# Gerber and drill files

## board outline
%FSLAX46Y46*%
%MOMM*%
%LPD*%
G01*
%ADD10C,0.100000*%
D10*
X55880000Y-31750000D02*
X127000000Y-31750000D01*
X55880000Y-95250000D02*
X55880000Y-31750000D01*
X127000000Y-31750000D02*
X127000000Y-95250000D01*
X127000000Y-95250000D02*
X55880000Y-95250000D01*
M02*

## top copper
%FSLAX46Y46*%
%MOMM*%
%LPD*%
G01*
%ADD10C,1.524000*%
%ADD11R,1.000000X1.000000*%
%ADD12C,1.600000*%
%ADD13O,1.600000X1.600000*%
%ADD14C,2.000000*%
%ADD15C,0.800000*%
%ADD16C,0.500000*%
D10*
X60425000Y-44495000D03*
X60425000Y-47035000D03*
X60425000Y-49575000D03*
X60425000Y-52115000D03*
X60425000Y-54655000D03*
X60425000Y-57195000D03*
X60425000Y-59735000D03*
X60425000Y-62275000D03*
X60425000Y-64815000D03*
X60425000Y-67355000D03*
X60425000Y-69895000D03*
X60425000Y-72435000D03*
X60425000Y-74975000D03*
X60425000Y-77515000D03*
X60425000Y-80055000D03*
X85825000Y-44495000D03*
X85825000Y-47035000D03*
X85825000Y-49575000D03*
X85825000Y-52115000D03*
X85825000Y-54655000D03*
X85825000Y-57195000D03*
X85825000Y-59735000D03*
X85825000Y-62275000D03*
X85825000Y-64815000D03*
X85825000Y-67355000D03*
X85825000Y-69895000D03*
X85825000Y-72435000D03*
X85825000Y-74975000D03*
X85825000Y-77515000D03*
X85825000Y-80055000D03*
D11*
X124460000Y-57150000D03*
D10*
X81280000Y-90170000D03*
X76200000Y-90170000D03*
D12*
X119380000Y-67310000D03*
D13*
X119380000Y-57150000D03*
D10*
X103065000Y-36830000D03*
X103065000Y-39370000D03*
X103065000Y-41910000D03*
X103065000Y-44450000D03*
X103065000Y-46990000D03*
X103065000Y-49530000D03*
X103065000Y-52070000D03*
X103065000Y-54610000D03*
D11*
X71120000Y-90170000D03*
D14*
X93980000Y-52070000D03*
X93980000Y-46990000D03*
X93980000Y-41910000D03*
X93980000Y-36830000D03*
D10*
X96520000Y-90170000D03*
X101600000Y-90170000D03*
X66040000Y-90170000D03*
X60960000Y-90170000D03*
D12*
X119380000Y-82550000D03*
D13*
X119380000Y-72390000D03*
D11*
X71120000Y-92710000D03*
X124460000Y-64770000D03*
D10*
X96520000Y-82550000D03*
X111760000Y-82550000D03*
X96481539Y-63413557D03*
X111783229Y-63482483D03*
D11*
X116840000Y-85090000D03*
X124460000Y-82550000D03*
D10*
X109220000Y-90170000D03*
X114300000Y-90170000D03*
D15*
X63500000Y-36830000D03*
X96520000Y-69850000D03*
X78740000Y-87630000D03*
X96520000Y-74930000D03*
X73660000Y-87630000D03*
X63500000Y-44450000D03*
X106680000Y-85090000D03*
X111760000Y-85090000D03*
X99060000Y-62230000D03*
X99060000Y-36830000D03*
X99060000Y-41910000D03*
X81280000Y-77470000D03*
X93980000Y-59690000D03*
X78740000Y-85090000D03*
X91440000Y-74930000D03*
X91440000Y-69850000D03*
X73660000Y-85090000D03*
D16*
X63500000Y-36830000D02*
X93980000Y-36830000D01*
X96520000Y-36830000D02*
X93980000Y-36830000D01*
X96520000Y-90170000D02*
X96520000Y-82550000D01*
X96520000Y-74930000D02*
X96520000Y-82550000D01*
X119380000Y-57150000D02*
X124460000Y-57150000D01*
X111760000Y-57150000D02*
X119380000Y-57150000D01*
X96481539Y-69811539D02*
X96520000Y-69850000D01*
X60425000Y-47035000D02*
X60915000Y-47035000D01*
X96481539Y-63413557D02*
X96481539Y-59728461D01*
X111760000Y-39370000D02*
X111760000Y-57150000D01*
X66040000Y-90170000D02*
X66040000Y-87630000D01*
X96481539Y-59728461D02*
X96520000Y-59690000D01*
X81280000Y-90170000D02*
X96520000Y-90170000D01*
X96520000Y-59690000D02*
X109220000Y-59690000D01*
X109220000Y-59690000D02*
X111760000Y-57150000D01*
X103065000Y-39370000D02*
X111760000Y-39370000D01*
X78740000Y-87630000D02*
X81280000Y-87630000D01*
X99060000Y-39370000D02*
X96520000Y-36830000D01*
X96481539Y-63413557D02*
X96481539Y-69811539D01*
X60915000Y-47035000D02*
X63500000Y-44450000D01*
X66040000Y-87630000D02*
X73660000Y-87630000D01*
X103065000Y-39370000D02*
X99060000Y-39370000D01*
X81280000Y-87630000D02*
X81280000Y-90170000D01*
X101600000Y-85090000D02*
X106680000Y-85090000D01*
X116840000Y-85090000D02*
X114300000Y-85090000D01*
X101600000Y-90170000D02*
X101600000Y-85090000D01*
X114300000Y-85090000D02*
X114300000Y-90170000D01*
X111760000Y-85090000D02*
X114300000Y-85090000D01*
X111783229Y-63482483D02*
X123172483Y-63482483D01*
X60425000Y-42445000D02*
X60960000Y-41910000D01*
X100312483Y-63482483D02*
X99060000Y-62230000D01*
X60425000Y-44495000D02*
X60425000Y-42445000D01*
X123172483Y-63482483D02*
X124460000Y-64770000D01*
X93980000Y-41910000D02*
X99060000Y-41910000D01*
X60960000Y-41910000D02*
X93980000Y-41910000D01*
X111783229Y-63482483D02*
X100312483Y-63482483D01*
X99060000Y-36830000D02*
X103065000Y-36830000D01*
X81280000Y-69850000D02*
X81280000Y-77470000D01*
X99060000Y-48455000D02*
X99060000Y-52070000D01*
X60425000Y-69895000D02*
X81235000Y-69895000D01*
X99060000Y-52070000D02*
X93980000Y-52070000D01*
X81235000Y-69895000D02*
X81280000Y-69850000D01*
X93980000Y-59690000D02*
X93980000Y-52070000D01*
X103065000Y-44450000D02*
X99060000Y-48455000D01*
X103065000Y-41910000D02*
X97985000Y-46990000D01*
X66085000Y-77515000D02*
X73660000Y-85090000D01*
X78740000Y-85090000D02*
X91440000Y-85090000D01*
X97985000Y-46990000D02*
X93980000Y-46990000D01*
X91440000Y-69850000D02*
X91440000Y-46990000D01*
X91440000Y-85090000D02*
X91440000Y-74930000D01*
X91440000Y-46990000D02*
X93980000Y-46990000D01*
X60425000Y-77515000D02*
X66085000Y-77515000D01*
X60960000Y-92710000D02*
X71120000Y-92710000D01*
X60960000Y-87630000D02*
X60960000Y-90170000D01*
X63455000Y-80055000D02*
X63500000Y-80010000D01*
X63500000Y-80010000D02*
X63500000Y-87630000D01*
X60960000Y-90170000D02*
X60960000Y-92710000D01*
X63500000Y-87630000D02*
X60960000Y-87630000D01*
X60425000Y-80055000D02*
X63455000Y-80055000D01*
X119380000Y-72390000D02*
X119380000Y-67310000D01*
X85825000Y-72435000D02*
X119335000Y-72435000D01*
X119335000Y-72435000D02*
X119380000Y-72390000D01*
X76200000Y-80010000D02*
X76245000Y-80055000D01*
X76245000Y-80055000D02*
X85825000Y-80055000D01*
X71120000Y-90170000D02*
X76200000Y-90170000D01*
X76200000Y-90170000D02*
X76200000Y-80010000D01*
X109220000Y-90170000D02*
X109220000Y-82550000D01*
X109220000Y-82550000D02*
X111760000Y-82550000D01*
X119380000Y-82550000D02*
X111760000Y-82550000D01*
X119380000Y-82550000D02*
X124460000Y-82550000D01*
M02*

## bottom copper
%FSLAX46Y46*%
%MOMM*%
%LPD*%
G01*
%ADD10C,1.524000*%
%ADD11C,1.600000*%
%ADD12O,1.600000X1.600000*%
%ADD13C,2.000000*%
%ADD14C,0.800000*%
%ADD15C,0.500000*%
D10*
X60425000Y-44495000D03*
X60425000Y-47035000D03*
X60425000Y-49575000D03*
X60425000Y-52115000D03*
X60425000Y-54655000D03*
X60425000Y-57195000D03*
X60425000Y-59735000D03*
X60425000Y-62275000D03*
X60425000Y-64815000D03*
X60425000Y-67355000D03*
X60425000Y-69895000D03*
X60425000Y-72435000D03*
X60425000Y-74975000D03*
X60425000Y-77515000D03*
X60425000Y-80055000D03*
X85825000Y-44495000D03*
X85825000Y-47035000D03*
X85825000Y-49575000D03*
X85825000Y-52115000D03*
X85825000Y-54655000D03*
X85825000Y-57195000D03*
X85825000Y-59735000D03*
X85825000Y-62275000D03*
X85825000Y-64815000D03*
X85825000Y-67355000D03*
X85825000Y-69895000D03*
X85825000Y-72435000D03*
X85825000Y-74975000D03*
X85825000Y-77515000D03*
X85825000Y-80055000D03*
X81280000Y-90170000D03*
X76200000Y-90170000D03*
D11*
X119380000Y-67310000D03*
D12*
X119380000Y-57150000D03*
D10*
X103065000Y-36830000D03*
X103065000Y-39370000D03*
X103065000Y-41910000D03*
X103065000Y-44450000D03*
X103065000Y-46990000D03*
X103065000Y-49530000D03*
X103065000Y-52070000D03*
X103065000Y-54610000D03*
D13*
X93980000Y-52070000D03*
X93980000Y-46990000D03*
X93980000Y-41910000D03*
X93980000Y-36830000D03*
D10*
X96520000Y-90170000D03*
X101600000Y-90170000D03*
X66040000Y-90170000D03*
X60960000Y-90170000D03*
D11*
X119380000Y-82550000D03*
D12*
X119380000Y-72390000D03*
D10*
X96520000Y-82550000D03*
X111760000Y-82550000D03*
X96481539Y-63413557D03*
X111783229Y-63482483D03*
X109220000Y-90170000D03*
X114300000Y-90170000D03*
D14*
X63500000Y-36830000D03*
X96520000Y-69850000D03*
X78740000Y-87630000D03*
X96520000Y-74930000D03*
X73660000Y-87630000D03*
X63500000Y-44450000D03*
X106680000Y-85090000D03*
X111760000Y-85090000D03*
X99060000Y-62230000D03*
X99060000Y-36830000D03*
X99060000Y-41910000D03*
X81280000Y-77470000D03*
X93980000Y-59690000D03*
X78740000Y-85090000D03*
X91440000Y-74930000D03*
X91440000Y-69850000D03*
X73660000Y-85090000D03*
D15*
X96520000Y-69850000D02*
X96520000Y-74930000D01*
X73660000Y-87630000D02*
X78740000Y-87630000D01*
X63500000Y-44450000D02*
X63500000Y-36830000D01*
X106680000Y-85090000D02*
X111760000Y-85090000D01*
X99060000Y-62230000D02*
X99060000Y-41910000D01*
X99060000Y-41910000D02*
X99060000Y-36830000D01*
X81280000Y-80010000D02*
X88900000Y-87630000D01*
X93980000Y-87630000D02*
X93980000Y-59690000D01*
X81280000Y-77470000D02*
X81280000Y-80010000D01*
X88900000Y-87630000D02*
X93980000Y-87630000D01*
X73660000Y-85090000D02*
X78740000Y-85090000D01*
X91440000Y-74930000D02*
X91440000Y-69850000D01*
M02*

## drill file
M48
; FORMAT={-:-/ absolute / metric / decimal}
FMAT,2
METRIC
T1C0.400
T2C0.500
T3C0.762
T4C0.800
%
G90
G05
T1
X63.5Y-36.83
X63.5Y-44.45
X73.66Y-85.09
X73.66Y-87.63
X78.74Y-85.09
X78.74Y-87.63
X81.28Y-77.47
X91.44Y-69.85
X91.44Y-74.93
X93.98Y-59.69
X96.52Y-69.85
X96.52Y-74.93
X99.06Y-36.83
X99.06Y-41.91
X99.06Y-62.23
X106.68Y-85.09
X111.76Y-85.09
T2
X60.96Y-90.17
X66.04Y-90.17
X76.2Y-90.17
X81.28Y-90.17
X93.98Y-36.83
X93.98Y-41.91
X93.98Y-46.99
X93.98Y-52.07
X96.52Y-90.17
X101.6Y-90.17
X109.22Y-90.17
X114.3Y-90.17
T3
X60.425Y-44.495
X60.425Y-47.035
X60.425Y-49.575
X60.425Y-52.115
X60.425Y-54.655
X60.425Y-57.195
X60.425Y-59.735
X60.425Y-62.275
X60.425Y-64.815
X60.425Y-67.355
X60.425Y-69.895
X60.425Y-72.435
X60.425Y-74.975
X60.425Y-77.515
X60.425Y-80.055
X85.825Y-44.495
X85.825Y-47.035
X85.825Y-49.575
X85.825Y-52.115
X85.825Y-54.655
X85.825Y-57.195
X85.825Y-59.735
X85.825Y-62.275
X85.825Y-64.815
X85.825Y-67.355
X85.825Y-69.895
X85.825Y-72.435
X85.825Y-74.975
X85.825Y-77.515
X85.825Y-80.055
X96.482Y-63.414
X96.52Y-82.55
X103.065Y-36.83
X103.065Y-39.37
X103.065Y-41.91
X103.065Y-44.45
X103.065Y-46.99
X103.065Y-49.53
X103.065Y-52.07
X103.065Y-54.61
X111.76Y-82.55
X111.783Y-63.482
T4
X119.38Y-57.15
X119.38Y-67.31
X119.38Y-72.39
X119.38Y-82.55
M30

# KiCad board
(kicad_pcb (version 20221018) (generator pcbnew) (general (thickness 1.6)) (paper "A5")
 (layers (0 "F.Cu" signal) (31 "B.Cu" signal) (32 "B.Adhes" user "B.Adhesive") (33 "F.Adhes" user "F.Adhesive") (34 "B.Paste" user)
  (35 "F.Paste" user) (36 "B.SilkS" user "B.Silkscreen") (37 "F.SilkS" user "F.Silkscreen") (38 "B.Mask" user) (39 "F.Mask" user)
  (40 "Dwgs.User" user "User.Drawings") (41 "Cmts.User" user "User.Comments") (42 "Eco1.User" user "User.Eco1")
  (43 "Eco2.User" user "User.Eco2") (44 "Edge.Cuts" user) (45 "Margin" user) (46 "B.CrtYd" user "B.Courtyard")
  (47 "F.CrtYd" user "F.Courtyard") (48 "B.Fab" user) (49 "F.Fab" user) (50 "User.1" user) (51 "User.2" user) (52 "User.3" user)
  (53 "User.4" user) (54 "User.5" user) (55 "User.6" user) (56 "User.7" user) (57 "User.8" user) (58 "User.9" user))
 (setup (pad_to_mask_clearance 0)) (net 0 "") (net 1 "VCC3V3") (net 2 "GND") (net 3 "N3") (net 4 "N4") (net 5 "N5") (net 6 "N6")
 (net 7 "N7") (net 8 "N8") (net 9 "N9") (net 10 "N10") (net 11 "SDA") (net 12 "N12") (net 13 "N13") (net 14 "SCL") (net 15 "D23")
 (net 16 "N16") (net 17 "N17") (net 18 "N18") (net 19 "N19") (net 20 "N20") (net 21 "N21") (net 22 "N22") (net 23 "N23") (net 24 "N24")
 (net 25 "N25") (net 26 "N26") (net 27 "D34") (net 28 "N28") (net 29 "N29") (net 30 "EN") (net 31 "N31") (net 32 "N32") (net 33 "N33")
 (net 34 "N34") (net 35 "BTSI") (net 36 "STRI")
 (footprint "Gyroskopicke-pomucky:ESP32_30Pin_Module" (layer "F.Cu") (at 78.205 67.355)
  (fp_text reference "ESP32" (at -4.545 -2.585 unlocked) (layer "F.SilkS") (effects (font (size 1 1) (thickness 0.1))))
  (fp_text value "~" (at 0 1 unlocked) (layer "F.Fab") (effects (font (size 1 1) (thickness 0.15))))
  (pad "1" thru_hole circle (at -17.78 -22.86) (size 1.524 1.524) (drill 0.762) (layers "*.Cu" "*.Mask") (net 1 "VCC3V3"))
  (pad "2" thru_hole circle (at -17.78 -20.32) (size 1.524 1.524) (drill 0.762) (layers "*.Cu" "*.Mask") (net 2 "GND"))
  (pad "3" thru_hole circle (at -17.78 -17.78) (size 1.524 1.524) (drill 0.762) (layers "*.Cu" "*.Mask") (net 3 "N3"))
  (pad "4" thru_hole circle (at -17.78 -15.24) (size 1.524 1.524) (drill 0.762) (layers "*.Cu" "*.Mask") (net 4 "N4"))
  (pad "5" thru_hole circle (at -17.78 -12.7) (size 1.524 1.524) (drill 0.762) (layers "*.Cu" "*.Mask") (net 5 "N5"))
  (pad "6" thru_hole circle (at -17.78 -10.16) (size 1.524 1.524) (drill 0.762) (layers "*.Cu" "*.Mask") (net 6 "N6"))
  (pad "7" thru_hole circle (at -17.78 -7.62) (size 1.524 1.524) (drill 0.762) (layers "*.Cu" "*.Mask") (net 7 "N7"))
  (pad "8" thru_hole circle (at -17.78 -5.08) (size 1.524 1.524) (drill 0.762) (layers "*.Cu" "*.Mask") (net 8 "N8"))
  (pad "9" thru_hole circle (at -17.78 -2.54) (size 1.524 1.524) (drill 0.762) (layers "*.Cu" "*.Mask") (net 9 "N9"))
  (pad "10" thru_hole circle (at -17.78 0) (size 1.524 1.524) (drill 0.762) (layers "*.Cu" "*.Mask") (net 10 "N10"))
  (pad "11" thru_hole circle (at -17.78 2.54) (size 1.524 1.524) (drill 0.762) (layers "*.Cu" "*.Mask") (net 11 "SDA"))
  (pad "12" thru_hole circle (at -17.78 5.08) (size 1.524 1.524) (drill 0.762) (layers "*.Cu" "*.Mask") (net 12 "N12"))
  (pad "13" thru_hole circle (at -17.78 7.62) (size 1.524 1.524) (drill 0.762) (layers "*.Cu" "*.Mask") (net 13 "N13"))
  (pad "14" thru_hole circle (at -17.78 10.16) (size 1.524 1.524) (drill 0.762) (layers "*.Cu" "*.Mask") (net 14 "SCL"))
  (pad "15" thru_hole circle (at -17.78 12.7) (size 1.524 1.524) (drill 0.762) (layers "*.Cu" "*.Mask") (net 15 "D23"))
  (pad "16" thru_hole circle (at 7.62 -22.86) (size 1.524 1.524) (drill 0.762) (layers "*.Cu" "*.Mask") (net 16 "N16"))
  (pad "17" thru_hole circle (at 7.62 -20.32) (size 1.524 1.524) (drill 0.762) (layers "*.Cu" "*.Mask") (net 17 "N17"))
  (pad "18" thru_hole circle (at 7.62 -17.78) (size 1.524 1.524) (drill 0.762) (layers "*.Cu" "*.Mask") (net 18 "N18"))
  (pad "19" thru_hole circle (at 7.62 -15.24) (size 1.524 1.524) (drill 0.762) (layers "*.Cu" "*.Mask") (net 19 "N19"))
  (pad "20" thru_hole circle (at 7.62 -12.7) (size 1.524 1.524) (drill 0.762) (layers "*.Cu" "*.Mask") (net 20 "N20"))
  (pad "21" thru_hole circle (at 7.62 -10.16) (size 1.524 1.524) (drill 0.762) (layers "*.Cu" "*.Mask") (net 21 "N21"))
  (pad "22" thru_hole circle (at 7.62 -7.62) (size 1.524 1.524) (drill 0.762) (layers "*.Cu" "*.Mask") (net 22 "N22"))
  (pad "23" thru_hole circle (at 7.62 -5.08) (size 1.524 1.524) (drill 0.762) (layers "*.Cu" "*.Mask") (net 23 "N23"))
  (pad "24" thru_hole circle (at 7.62 -2.54) (size 1.524 1.524) (drill 0.762) (layers "*.Cu" "*.Mask") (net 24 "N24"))
  (pad "25" thru_hole circle (at 7.62 0) (size 1.524 1.524) (drill 0.762) (layers "*.Cu" "*.Mask") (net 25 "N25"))
  (pad "26" thru_hole circle (at 7.62 2.54) (size 1.524 1.524) (drill 0.762) (layers "*.Cu" "*.Mask") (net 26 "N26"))
  (pad "27" thru_hole circle (at 7.62 5.08) (size 1.524 1.524) (drill 0.762) (layers "*.Cu" "*.Mask") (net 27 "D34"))
  (pad "28" thru_hole circle (at 7.62 7.62) (size 1.524 1.524) (drill 0.762) (layers "*.Cu" "*.Mask") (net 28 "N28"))
  (pad "29" thru_hole circle (at 7.62 10.16) (size 1.524 1.524) (drill 0.762) (layers "*.Cu" "*.Mask") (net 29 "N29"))
  (pad "30" thru_hole circle (at 7.62 12.7) (size 1.524 1.524) (drill 0.762) (layers "*.Cu" "*.Mask") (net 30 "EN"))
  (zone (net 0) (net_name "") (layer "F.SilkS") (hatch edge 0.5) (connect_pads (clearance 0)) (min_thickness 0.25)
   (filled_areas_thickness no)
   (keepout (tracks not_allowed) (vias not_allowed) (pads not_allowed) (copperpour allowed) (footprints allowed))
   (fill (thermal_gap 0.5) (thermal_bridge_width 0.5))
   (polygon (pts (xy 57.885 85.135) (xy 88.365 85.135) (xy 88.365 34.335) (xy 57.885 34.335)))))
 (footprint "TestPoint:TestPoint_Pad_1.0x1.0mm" (layer "F.Cu") (at 124.46 57.15)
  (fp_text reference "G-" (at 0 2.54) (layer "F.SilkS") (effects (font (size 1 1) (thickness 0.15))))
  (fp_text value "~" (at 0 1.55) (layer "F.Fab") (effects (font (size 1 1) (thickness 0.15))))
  (pad "1" smd rect (at 0 0) (size 1 1) (layers "F.Cu" "F.Mask") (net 2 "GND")))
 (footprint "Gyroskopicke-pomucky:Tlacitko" (layer "F.Cu") (at 78.74 90.17 180)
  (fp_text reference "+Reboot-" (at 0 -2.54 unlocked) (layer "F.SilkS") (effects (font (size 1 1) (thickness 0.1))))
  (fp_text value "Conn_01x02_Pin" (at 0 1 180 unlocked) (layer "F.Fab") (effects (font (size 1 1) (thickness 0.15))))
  (pad "1" thru_hole circle (at -2.54 0 180) (size 1.524 1.524) (drill 0.5) (layers "*.Cu" "*.Mask") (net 2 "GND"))
  (pad "2" thru_hole circle (at 2.54 0 180) (size 1.524 1.524) (drill 0.5) (layers "*.Cu" "*.Mask") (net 30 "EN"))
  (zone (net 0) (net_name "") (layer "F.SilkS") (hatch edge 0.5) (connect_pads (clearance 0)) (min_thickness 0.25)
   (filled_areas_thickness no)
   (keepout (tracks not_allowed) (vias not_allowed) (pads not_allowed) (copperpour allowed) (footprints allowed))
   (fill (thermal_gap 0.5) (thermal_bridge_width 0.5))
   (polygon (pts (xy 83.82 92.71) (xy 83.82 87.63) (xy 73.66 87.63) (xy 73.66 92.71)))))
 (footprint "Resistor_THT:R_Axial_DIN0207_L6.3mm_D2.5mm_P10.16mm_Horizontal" (layer "F.Cu") (at 119.38 67.31 90)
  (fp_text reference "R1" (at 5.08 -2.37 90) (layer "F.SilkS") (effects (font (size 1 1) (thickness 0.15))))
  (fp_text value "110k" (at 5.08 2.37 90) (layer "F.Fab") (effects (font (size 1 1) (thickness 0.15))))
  (pad "1" thru_hole circle (at 0 0 90) (size 1.6 1.6) (drill 0.8) (layers "*.Cu" "*.Mask") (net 27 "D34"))
  (pad "2" thru_hole oval (at 10.16 0 90) (size 1.6 1.6) (drill 0.8) (layers "*.Cu" "*.Mask") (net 2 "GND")))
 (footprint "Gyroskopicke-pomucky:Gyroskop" (layer "F.Cu") (at 108.145 44.45)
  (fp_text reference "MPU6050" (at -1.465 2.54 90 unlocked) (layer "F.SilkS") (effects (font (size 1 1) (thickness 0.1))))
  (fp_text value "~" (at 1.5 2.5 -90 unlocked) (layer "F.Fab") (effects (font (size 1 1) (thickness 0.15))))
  (pad "1" thru_hole circle (at -5.08 -7.62 270) (size 1.524 1.524) (drill 0.762) (layers "*.Cu" "*.Mask") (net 1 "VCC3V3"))
  (pad "2" thru_hole circle (at -5.08 -5.08 270) (size 1.524 1.524) (drill 0.762) (layers "*.Cu" "*.Mask") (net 2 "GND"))
  (pad "3" thru_hole circle (at -5.08 -2.54 270) (size 1.524 1.524) (drill 0.762) (layers "*.Cu" "*.Mask") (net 14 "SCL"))
  (pad "4" thru_hole circle (at -5.08 0 270) (size 1.524 1.524) (drill 0.762) (layers "*.Cu" "*.Mask") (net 11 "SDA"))
  (pad "5" thru_hole circle (at -5.08 2.54 270) (size 1.524 1.524) (drill 0.762) (layers "*.Cu" "*.Mask") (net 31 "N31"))
  (pad "6" thru_hole circle (at -5.08 5.08 270) (size 1.524 1.524) (drill 0.762) (layers "*.Cu" "*.Mask") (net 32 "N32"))
  (pad "7" thru_hole circle (at -5.08 7.62 270) (size 1.524 1.524) (drill 0.762) (layers "*.Cu" "*.Mask") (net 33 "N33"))
  (pad "8" thru_hole circle (at -5.08 10.16 270) (size 1.524 1.524) (drill 0.762) (layers "*.Cu" "*.Mask") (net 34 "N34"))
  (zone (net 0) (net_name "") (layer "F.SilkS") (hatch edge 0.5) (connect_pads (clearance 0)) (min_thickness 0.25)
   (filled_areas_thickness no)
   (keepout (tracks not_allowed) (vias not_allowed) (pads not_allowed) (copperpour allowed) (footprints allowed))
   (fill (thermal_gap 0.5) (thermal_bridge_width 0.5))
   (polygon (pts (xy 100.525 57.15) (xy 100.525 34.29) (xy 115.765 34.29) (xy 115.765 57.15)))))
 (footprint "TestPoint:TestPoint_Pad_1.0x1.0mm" (layer "F.Cu") (at 71.12 90.17)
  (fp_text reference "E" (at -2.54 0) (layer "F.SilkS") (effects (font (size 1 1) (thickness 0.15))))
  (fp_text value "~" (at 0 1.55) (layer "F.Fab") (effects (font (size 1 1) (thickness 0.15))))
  (pad "1" smd rect (at 0 0) (size 1 1) (layers "F.Cu" "F.Mask") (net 30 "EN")))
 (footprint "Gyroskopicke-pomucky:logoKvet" (layer "F.Cu") (at 121.92 90.17)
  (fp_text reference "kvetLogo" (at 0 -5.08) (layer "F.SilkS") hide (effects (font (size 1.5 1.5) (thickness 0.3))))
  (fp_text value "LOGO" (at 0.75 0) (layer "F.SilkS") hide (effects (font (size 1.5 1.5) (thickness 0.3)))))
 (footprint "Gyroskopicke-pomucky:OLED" (layer "F.Cu") (at 93.98 44.45 90)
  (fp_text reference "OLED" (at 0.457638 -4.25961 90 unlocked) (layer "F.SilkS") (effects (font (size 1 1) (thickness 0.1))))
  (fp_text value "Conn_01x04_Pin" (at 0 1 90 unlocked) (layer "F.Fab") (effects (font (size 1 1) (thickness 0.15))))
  (pad "1" thru_hole circle (at -7.62 0 90) (size 2 2) (drill 0.5) (layers "*.Cu" "*.Mask") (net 11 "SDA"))
  (pad "2" thru_hole circle (at -2.54 0 90) (size 2 2) (drill 0.5) (layers "*.Cu" "*.Mask") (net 14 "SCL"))
  (pad "3" thru_hole circle (at 2.54 0 90) (size 2 2) (drill 0.5) (layers "*.Cu" "*.Mask") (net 1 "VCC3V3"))
  (pad "4" thru_hole circle (at 7.62 0 90) (size 2 2) (drill 0.5) (layers "*.Cu" "*.Mask") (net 2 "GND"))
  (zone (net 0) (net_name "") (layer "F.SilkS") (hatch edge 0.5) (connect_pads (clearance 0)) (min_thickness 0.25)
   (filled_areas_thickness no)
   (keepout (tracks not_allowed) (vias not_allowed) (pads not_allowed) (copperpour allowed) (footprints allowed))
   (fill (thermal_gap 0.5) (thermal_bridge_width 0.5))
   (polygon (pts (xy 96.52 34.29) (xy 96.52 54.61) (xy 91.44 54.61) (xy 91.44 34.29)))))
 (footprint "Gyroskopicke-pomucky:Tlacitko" (layer "F.Cu") (at 99.06 90.17)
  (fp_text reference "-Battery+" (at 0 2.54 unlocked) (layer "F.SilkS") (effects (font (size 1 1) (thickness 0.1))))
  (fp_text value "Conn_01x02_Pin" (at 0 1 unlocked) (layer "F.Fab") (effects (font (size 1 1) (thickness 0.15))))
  (pad "1" thru_hole circle (at -2.54 0) (size 1.524 1.524) (drill 0.5) (layers "*.Cu" "*.Mask") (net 2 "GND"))
  (pad "2" thru_hole circle (at 2.54 0) (size 1.524 1.524) (drill 0.5) (layers "*.Cu" "*.Mask") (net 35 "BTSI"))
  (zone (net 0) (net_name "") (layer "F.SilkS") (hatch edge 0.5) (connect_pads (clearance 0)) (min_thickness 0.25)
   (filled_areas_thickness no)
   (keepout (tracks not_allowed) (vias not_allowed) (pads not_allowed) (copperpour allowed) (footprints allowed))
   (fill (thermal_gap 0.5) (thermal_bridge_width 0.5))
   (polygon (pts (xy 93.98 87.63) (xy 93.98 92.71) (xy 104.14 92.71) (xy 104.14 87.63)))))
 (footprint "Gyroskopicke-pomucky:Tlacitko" (layer "F.Cu") (at 63.5 90.17 180)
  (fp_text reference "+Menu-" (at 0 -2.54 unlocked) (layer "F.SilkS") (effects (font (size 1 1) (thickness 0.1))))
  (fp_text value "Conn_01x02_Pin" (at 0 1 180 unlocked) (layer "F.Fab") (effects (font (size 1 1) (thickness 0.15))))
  (pad "1" thru_hole circle (at -2.54 0 180) (size 1.524 1.524) (drill 0.5) (layers "*.Cu" "*.Mask") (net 2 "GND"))
  (pad "2" thru_hole circle (at 2.54 0 180) (size 1.524 1.524) (drill 0.5) (layers "*.Cu" "*.Mask") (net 15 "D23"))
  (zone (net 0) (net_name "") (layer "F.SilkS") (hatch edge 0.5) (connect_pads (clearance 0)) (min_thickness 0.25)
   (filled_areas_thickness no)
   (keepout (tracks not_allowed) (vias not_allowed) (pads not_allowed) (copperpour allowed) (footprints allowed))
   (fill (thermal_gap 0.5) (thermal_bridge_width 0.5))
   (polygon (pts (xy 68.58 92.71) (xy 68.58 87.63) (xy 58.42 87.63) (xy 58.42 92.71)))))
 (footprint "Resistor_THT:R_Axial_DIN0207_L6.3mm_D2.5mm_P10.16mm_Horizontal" (layer "F.Cu") (at 119.38 82.55 90)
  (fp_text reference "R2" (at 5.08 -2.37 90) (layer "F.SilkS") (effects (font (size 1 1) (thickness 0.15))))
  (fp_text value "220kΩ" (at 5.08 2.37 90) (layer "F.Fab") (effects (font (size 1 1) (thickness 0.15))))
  (pad "1" thru_hole circle (at 0 0 90) (size 1.6 1.6) (drill 0.8) (layers "*.Cu" "*.Mask") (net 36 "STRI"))
  (pad "2" thru_hole oval (at 10.16 0 90) (size 1.6 1.6) (drill 0.8) (layers "*.Cu" "*.Mask") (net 27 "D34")))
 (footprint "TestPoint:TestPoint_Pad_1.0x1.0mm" (layer "F.Cu") (at 71.12 92.71)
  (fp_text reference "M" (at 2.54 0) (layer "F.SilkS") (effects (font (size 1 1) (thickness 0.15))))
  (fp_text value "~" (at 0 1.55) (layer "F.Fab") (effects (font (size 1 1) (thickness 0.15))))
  (pad "1" smd rect (at 0 0) (size 1 1) (layers "F.Cu" "F.Mask") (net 15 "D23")))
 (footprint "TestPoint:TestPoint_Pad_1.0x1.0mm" (layer "F.Cu") (at 124.46 64.77)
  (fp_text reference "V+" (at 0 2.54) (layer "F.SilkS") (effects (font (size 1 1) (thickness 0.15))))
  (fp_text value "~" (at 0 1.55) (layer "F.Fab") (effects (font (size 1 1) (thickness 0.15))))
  (pad "1" smd rect (at 0 0) (size 1 1) (layers "F.Cu" "F.Mask") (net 1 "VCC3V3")))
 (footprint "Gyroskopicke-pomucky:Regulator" (layer "F.Cu") (at 106.68 72.39 90)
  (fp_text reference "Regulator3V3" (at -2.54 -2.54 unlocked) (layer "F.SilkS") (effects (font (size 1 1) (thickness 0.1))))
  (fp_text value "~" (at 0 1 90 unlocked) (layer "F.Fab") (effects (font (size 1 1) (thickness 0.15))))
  (pad "1" thru_hole circle (at -10.16 -10.16 90) (size 1.524 1.524) (drill 0.762) (layers "*.Cu" "*.Mask") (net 2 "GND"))
  (pad "2" thru_hole circle (at -10.16 5.08 90) (size 1.524 1.524) (drill 0.762) (layers "*.Cu" "*.Mask") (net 36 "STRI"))
  (pad "3" thru_hole circle (at 8.976443 -10.198461 90) (size 1.524 1.524) (drill 0.762) (layers "*.Cu" "*.Mask") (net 2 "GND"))
  (pad "4" thru_hole circle (at 8.907517 5.103229 90) (size 1.524 1.524) (drill 0.762) (layers "*.Cu" "*.Mask") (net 1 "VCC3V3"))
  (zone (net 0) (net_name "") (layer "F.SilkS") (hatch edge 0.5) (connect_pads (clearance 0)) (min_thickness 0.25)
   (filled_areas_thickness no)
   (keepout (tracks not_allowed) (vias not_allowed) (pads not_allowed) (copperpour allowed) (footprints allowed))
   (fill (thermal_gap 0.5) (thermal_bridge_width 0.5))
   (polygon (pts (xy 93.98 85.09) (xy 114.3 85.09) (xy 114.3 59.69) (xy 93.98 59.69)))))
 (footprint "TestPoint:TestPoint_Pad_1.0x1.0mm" (layer "F.Cu") (at 116.84 85.09)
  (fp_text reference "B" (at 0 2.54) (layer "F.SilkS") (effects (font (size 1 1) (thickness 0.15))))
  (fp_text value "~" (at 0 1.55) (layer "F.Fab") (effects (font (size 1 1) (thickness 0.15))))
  (pad "1" smd rect (at 0 0) (size 1 1) (layers "F.Cu" "F.Mask") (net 35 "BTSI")))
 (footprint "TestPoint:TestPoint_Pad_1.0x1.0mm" (layer "F.Cu") (at 124.46 82.55)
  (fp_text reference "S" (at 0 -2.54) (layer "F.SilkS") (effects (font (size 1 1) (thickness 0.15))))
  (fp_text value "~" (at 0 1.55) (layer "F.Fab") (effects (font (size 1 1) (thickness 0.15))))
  (pad "1" smd rect (at 0 0) (size 1 1) (layers "F.Cu" "F.Mask") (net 36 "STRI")))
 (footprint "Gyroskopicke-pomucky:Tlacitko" (layer "F.Cu") (at 111.76 90.17)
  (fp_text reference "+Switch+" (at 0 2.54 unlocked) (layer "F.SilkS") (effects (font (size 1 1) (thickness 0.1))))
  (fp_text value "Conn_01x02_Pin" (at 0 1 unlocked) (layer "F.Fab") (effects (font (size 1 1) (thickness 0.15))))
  (pad "1" thru_hole circle (at -2.54 0) (size 1.524 1.524) (drill 0.5) (layers "*.Cu" "*.Mask") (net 36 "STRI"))
  (pad "2" thru_hole circle (at 2.54 0) (size 1.524 1.524) (drill 0.5) (layers "*.Cu" "*.Mask") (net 35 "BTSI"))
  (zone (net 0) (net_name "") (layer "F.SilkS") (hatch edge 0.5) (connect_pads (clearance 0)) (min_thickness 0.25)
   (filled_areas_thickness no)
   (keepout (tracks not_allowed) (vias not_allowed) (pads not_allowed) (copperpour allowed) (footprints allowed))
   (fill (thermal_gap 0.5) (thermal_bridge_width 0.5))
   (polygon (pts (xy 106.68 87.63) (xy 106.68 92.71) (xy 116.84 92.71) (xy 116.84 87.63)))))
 (gr_line (start 55.88 31.75) (end 127 31.75) (stroke (width 0.1) (type default)) (layer "Edge.Cuts"))
 (gr_line (start 55.88 95.25) (end 55.88 31.75) (stroke (width 0.1) (type default)) (layer "Edge.Cuts"))
 (gr_line (start 127 31.75) (end 127 95.25) (stroke (width 0.1) (type default)) (layer "Edge.Cuts"))
 (gr_line (start 127 95.25) (end 55.88 95.25) (stroke (width 0.1) (type default)) (layer "Edge.Cuts"))
 (segment (start 63.5 36.83) (end 93.98 36.83) (width 0.5) (layer "F.Cu") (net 2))
 (segment (start 96.52 36.83) (end 93.98 36.83) (width 0.5) (layer "F.Cu") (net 2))
 (segment (start 96.52 90.17) (end 96.52 82.55) (width 0.5) (layer "F.Cu") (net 2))
 (segment (start 96.52 74.93) (end 96.52 82.55) (width 0.5) (layer "F.Cu") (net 2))
 (segment (start 119.38 57.15) (end 124.46 57.15) (width 0.5) (layer "F.Cu") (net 2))
 (segment (start 111.76 57.15) (end 119.38 57.15) (width 0.5) (layer "F.Cu") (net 2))
 (segment (start 96.481539 69.811539) (end 96.52 69.85) (width 0.5) (layer "F.Cu") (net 2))
 (segment (start 60.425 47.035) (end 60.915 47.035) (width 0.5) (layer "F.Cu") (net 2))
 (segment (start 96.481539 63.413557) (end 96.481539 59.728461) (width 0.5) (layer "F.Cu") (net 2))
 (segment (start 111.76 39.37) (end 111.76 57.15) (width 0.5) (layer "F.Cu") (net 2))
 (segment (start 66.04 90.17) (end 66.04 87.63) (width 0.5) (layer "F.Cu") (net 2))
 (segment (start 96.481539 59.728461) (end 96.52 59.69) (width 0.5) (layer "F.Cu") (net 2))
 (segment (start 81.28 90.17) (end 96.52 90.17) (width 0.5) (layer "F.Cu") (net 2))
 (segment (start 96.52 59.69) (end 109.22 59.69) (width 0.5) (layer "F.Cu") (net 2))
 (segment (start 109.22 59.69) (end 111.76 57.15) (width 0.5) (layer "F.Cu") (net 2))
 (segment (start 103.065 39.37) (end 111.76 39.37) (width 0.5) (layer "F.Cu") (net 2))
 (segment (start 78.74 87.63) (end 81.28 87.63) (width 0.5) (layer "F.Cu") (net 2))
 (segment (start 99.06 39.37) (end 96.52 36.83) (width 0.5) (layer "F.Cu") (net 2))
 (segment (start 96.481539 63.413557) (end 96.481539 69.811539) (width 0.5) (layer "F.Cu") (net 2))
 (segment (start 60.915 47.035) (end 63.5 44.45) (width 0.5) (layer "F.Cu") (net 2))
 (segment (start 66.04 87.63) (end 73.66 87.63) (width 0.5) (layer "F.Cu") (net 2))
 (segment (start 103.065 39.37) (end 99.06 39.37) (width 0.5) (layer "F.Cu") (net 2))
 (segment (start 81.28 87.63) (end 81.28 90.17) (width 0.5) (layer "F.Cu") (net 2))
 (via (at 63.5 36.83) (size 0.8) (drill 0.4) (layers "F.Cu" "B.Cu") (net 2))
 (via (at 96.52 69.85) (size 0.8) (drill 0.4) (layers "F.Cu" "B.Cu") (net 2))
 (via (at 78.74 87.63) (size 0.8) (drill 0.4) (layers "F.Cu" "B.Cu") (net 2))
 (via (at 96.52 74.93) (size 0.8) (drill 0.4) (layers "F.Cu" "B.Cu") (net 2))
 (via (at 73.66 87.63) (size 0.8) (drill 0.4) (layers "F.Cu" "B.Cu") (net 2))
 (via (at 63.5 44.45) (size 0.8) (drill 0.4) (layers "F.Cu" "B.Cu") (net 2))
 (segment (start 96.52 69.85) (end 96.52 74.93) (width 0.5) (layer "B.Cu") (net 2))
 (segment (start 73.66 87.63) (end 78.74 87.63) (width 0.5) (layer "B.Cu") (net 2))
 (segment (start 63.5 44.45) (end 63.5 36.83) (width 0.5) (layer "B.Cu") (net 2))
 (segment (start 101.6 85.09) (end 106.68 85.09) (width 0.5) (layer "F.Cu") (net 35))
 (segment (start 116.84 85.09) (end 114.3 85.09) (width 0.5) (layer "F.Cu") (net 35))
 (segment (start 101.6 90.17) (end 101.6 85.09) (width 0.5) (layer "F.Cu") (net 35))
 (segment (start 114.3 85.09) (end 114.3 90.17) (width 0.5) (layer "F.Cu") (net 35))
 (segment (start 111.76 85.09) (end 114.3 85.09) (width 0.5) (layer "F.Cu") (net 35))
 (via (at 106.68 85.09) (size 0.8) (drill 0.4) (layers "F.Cu" "B.Cu") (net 35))
 (via (at 111.76 85.09) (size 0.8) (drill 0.4) (layers "F.Cu" "B.Cu") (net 35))
 (segment (start 106.68 85.09) (end 111.76 85.09) (width 0.5) (layer "B.Cu") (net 35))
 (segment (start 111.783229 63.482483) (end 123.172483 63.482483) (width 0.5) (layer "F.Cu") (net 1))
 (segment (start 60.425 42.445) (end 60.96 41.91) (width 0.5) (layer "F.Cu") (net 1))
 (segment (start 100.312483 63.482483) (end 99.06 62.23) (width 0.5) (layer "F.Cu") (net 1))
 (segment (start 60.425 44.495) (end 60.425 42.445) (width 0.5) (layer "F.Cu") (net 1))
 (segment (start 123.172483 63.482483) (end 124.46 64.77) (width 0.5) (layer "F.Cu") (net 1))
 (segment (start 93.98 41.91) (end 99.06 41.91) (width 0.5) (layer "F.Cu") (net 1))
 (segment (start 60.96 41.91) (end 93.98 41.91) (width 0.5) (layer "F.Cu") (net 1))
 (segment (start 111.783229 63.482483) (end 100.312483 63.482483) (width 0.5) (layer "F.Cu") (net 1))
 (segment (start 99.06 36.83) (end 103.065 36.83) (width 0.5) (layer "F.Cu") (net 1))
 (via (at 99.06 62.23) (size 0.8) (drill 0.4) (layers "F.Cu" "B.Cu") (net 1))
 (via (at 99.06 36.83) (size 0.8) (drill 0.4) (layers "F.Cu" "B.Cu") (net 1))
 (via (at 99.06 41.91) (size 0.8) (drill 0.4) (layers "F.Cu" "B.Cu") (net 1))
 (segment (start 99.06 62.23) (end 99.06 41.91) (width 0.5) (layer "B.Cu") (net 1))
 (segment (start 99.06 41.91) (end 99.06 36.83) (width 0.5) (layer "B.Cu") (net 1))
 (segment (start 81.28 69.85) (end 81.28 77.47) (width 0.5) (layer "F.Cu") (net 11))
 (segment (start 99.06 48.455) (end 99.06 52.07) (width 0.5) (layer "F.Cu") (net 11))
 (segment (start 60.425 69.895) (end 81.235 69.895) (width 0.5) (layer "F.Cu") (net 11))
 (segment (start 99.06 52.07) (end 93.98 52.07) (width 0.5) (layer "F.Cu") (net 11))
 (segment (start 81.235 69.895) (end 81.28 69.85) (width 0.5) (layer "F.Cu") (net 11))
 (segment (start 93.98 59.69) (end 93.98 52.07) (width 0.5) (layer "F.Cu") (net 11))
 (segment (start 103.065 44.45) (end 99.06 48.455) (width 0.5) (layer "F.Cu") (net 11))
 (via (at 81.28 77.47) (size 0.8) (drill 0.4) (layers "F.Cu" "B.Cu") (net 11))
 (via (at 93.98 59.69) (size 0.8) (drill 0.4) (layers "F.Cu" "B.Cu") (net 11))
 (segment (start 81.28 80.01) (end 88.9 87.63) (width 0.5) (layer "B.Cu") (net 11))
 (segment (start 93.98 87.63) (end 93.98 59.69) (width 0.5) (layer "B.Cu") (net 11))
 (segment (start 81.28 77.47) (end 81.28 80.01) (width 0.5) (layer "B.Cu") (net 11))
 (segment (start 88.9 87.63) (end 93.98 87.63) (width 0.5) (layer "B.Cu") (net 11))
 (segment (start 103.065 41.91) (end 97.985 46.99) (width 0.5) (layer "F.Cu") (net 14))
 (segment (start 66.085 77.515) (end 73.66 85.09) (width 0.5) (layer "F.Cu") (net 14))
 (segment (start 78.74 85.09) (end 91.44 85.09) (width 0.5) (layer "F.Cu") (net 14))
 (segment (start 97.985 46.99) (end 93.98 46.99) (width 0.5) (layer "F.Cu") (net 14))
 (segment (start 91.44 69.85) (end 91.44 46.99) (width 0.5) (layer "F.Cu") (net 14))
 (segment (start 91.44 85.09) (end 91.44 74.93) (width 0.5) (layer "F.Cu") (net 14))
 (segment (start 91.44 46.99) (end 93.98 46.99) (width 0.5) (layer "F.Cu") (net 14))
 (segment (start 60.425 77.515) (end 66.085 77.515) (width 0.5) (layer "F.Cu") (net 14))
 (via (at 78.74 85.09) (size 0.8) (drill 0.4) (layers "F.Cu" "B.Cu") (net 14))
 (via (at 91.44 74.93) (size 0.8) (drill 0.4) (layers "F.Cu" "B.Cu") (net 14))
 (via (at 91.44 69.85) (size 0.8) (drill 0.4) (layers "F.Cu" "B.Cu") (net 14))
 (via (at 73.66 85.09) (size 0.8) (drill 0.4) (layers "F.Cu" "B.Cu") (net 14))
 (segment (start 73.66 85.09) (end 78.74 85.09) (width 0.5) (layer "B.Cu") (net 14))
 (segment (start 91.44 74.93) (end 91.44 69.85) (width 0.5) (layer "B.Cu") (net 14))
 (segment (start 60.96 92.71) (end 71.12 92.71) (width 0.5) (layer "F.Cu") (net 15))
 (segment (start 60.96 87.63) (end 60.96 90.17) (width 0.5) (layer "F.Cu") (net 15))
 (segment (start 63.455 80.055) (end 63.5 80.01) (width 0.5) (layer "F.Cu") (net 15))
 (segment (start 63.5 80.01) (end 63.5 87.63) (width 0.5) (layer "F.Cu") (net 15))
 (segment (start 60.96 90.17) (end 60.96 92.71) (width 0.5) (layer "F.Cu") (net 15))
 (segment (start 63.5 87.63) (end 60.96 87.63) (width 0.5) (layer "F.Cu") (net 15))
 (segment (start 60.425 80.055) (end 63.455 80.055) (width 0.5) (layer "F.Cu") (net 15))
 (segment (start 119.38 72.39) (end 119.38 67.31) (width 0.5) (layer "F.Cu") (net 27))
 (segment (start 85.825 72.435) (end 119.335 72.435) (width 0.5) (layer "F.Cu") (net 27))
 (segment (start 119.335 72.435) (end 119.38 72.39) (width 0.5) (layer "F.Cu") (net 27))
 (segment (start 76.2 80.01) (end 76.245 80.055) (width 0.5) (layer "F.Cu") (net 30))
 (segment (start 76.245 80.055) (end 85.825 80.055) (width 0.5) (layer "F.Cu") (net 30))
 (segment (start 71.12 90.17) (end 76.2 90.17) (width 0.5) (layer "F.Cu") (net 30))
 (segment (start 76.2 90.17) (end 76.2 80.01) (width 0.5) (layer "F.Cu") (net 30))
 (segment (start 109.22 90.17) (end 109.22 82.55) (width 0.5) (layer "F.Cu") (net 36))
 (segment (start 109.22 82.55) (end 111.76 82.55) (width 0.5) (layer "F.Cu") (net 36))
 (segment (start 119.38 82.55) (end 111.76 82.55) (width 0.5) (layer "F.Cu") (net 36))
 (segment (start 119.38 82.55) (end 124.46 82.55) (width 0.5) (layer "F.Cu") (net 36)))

